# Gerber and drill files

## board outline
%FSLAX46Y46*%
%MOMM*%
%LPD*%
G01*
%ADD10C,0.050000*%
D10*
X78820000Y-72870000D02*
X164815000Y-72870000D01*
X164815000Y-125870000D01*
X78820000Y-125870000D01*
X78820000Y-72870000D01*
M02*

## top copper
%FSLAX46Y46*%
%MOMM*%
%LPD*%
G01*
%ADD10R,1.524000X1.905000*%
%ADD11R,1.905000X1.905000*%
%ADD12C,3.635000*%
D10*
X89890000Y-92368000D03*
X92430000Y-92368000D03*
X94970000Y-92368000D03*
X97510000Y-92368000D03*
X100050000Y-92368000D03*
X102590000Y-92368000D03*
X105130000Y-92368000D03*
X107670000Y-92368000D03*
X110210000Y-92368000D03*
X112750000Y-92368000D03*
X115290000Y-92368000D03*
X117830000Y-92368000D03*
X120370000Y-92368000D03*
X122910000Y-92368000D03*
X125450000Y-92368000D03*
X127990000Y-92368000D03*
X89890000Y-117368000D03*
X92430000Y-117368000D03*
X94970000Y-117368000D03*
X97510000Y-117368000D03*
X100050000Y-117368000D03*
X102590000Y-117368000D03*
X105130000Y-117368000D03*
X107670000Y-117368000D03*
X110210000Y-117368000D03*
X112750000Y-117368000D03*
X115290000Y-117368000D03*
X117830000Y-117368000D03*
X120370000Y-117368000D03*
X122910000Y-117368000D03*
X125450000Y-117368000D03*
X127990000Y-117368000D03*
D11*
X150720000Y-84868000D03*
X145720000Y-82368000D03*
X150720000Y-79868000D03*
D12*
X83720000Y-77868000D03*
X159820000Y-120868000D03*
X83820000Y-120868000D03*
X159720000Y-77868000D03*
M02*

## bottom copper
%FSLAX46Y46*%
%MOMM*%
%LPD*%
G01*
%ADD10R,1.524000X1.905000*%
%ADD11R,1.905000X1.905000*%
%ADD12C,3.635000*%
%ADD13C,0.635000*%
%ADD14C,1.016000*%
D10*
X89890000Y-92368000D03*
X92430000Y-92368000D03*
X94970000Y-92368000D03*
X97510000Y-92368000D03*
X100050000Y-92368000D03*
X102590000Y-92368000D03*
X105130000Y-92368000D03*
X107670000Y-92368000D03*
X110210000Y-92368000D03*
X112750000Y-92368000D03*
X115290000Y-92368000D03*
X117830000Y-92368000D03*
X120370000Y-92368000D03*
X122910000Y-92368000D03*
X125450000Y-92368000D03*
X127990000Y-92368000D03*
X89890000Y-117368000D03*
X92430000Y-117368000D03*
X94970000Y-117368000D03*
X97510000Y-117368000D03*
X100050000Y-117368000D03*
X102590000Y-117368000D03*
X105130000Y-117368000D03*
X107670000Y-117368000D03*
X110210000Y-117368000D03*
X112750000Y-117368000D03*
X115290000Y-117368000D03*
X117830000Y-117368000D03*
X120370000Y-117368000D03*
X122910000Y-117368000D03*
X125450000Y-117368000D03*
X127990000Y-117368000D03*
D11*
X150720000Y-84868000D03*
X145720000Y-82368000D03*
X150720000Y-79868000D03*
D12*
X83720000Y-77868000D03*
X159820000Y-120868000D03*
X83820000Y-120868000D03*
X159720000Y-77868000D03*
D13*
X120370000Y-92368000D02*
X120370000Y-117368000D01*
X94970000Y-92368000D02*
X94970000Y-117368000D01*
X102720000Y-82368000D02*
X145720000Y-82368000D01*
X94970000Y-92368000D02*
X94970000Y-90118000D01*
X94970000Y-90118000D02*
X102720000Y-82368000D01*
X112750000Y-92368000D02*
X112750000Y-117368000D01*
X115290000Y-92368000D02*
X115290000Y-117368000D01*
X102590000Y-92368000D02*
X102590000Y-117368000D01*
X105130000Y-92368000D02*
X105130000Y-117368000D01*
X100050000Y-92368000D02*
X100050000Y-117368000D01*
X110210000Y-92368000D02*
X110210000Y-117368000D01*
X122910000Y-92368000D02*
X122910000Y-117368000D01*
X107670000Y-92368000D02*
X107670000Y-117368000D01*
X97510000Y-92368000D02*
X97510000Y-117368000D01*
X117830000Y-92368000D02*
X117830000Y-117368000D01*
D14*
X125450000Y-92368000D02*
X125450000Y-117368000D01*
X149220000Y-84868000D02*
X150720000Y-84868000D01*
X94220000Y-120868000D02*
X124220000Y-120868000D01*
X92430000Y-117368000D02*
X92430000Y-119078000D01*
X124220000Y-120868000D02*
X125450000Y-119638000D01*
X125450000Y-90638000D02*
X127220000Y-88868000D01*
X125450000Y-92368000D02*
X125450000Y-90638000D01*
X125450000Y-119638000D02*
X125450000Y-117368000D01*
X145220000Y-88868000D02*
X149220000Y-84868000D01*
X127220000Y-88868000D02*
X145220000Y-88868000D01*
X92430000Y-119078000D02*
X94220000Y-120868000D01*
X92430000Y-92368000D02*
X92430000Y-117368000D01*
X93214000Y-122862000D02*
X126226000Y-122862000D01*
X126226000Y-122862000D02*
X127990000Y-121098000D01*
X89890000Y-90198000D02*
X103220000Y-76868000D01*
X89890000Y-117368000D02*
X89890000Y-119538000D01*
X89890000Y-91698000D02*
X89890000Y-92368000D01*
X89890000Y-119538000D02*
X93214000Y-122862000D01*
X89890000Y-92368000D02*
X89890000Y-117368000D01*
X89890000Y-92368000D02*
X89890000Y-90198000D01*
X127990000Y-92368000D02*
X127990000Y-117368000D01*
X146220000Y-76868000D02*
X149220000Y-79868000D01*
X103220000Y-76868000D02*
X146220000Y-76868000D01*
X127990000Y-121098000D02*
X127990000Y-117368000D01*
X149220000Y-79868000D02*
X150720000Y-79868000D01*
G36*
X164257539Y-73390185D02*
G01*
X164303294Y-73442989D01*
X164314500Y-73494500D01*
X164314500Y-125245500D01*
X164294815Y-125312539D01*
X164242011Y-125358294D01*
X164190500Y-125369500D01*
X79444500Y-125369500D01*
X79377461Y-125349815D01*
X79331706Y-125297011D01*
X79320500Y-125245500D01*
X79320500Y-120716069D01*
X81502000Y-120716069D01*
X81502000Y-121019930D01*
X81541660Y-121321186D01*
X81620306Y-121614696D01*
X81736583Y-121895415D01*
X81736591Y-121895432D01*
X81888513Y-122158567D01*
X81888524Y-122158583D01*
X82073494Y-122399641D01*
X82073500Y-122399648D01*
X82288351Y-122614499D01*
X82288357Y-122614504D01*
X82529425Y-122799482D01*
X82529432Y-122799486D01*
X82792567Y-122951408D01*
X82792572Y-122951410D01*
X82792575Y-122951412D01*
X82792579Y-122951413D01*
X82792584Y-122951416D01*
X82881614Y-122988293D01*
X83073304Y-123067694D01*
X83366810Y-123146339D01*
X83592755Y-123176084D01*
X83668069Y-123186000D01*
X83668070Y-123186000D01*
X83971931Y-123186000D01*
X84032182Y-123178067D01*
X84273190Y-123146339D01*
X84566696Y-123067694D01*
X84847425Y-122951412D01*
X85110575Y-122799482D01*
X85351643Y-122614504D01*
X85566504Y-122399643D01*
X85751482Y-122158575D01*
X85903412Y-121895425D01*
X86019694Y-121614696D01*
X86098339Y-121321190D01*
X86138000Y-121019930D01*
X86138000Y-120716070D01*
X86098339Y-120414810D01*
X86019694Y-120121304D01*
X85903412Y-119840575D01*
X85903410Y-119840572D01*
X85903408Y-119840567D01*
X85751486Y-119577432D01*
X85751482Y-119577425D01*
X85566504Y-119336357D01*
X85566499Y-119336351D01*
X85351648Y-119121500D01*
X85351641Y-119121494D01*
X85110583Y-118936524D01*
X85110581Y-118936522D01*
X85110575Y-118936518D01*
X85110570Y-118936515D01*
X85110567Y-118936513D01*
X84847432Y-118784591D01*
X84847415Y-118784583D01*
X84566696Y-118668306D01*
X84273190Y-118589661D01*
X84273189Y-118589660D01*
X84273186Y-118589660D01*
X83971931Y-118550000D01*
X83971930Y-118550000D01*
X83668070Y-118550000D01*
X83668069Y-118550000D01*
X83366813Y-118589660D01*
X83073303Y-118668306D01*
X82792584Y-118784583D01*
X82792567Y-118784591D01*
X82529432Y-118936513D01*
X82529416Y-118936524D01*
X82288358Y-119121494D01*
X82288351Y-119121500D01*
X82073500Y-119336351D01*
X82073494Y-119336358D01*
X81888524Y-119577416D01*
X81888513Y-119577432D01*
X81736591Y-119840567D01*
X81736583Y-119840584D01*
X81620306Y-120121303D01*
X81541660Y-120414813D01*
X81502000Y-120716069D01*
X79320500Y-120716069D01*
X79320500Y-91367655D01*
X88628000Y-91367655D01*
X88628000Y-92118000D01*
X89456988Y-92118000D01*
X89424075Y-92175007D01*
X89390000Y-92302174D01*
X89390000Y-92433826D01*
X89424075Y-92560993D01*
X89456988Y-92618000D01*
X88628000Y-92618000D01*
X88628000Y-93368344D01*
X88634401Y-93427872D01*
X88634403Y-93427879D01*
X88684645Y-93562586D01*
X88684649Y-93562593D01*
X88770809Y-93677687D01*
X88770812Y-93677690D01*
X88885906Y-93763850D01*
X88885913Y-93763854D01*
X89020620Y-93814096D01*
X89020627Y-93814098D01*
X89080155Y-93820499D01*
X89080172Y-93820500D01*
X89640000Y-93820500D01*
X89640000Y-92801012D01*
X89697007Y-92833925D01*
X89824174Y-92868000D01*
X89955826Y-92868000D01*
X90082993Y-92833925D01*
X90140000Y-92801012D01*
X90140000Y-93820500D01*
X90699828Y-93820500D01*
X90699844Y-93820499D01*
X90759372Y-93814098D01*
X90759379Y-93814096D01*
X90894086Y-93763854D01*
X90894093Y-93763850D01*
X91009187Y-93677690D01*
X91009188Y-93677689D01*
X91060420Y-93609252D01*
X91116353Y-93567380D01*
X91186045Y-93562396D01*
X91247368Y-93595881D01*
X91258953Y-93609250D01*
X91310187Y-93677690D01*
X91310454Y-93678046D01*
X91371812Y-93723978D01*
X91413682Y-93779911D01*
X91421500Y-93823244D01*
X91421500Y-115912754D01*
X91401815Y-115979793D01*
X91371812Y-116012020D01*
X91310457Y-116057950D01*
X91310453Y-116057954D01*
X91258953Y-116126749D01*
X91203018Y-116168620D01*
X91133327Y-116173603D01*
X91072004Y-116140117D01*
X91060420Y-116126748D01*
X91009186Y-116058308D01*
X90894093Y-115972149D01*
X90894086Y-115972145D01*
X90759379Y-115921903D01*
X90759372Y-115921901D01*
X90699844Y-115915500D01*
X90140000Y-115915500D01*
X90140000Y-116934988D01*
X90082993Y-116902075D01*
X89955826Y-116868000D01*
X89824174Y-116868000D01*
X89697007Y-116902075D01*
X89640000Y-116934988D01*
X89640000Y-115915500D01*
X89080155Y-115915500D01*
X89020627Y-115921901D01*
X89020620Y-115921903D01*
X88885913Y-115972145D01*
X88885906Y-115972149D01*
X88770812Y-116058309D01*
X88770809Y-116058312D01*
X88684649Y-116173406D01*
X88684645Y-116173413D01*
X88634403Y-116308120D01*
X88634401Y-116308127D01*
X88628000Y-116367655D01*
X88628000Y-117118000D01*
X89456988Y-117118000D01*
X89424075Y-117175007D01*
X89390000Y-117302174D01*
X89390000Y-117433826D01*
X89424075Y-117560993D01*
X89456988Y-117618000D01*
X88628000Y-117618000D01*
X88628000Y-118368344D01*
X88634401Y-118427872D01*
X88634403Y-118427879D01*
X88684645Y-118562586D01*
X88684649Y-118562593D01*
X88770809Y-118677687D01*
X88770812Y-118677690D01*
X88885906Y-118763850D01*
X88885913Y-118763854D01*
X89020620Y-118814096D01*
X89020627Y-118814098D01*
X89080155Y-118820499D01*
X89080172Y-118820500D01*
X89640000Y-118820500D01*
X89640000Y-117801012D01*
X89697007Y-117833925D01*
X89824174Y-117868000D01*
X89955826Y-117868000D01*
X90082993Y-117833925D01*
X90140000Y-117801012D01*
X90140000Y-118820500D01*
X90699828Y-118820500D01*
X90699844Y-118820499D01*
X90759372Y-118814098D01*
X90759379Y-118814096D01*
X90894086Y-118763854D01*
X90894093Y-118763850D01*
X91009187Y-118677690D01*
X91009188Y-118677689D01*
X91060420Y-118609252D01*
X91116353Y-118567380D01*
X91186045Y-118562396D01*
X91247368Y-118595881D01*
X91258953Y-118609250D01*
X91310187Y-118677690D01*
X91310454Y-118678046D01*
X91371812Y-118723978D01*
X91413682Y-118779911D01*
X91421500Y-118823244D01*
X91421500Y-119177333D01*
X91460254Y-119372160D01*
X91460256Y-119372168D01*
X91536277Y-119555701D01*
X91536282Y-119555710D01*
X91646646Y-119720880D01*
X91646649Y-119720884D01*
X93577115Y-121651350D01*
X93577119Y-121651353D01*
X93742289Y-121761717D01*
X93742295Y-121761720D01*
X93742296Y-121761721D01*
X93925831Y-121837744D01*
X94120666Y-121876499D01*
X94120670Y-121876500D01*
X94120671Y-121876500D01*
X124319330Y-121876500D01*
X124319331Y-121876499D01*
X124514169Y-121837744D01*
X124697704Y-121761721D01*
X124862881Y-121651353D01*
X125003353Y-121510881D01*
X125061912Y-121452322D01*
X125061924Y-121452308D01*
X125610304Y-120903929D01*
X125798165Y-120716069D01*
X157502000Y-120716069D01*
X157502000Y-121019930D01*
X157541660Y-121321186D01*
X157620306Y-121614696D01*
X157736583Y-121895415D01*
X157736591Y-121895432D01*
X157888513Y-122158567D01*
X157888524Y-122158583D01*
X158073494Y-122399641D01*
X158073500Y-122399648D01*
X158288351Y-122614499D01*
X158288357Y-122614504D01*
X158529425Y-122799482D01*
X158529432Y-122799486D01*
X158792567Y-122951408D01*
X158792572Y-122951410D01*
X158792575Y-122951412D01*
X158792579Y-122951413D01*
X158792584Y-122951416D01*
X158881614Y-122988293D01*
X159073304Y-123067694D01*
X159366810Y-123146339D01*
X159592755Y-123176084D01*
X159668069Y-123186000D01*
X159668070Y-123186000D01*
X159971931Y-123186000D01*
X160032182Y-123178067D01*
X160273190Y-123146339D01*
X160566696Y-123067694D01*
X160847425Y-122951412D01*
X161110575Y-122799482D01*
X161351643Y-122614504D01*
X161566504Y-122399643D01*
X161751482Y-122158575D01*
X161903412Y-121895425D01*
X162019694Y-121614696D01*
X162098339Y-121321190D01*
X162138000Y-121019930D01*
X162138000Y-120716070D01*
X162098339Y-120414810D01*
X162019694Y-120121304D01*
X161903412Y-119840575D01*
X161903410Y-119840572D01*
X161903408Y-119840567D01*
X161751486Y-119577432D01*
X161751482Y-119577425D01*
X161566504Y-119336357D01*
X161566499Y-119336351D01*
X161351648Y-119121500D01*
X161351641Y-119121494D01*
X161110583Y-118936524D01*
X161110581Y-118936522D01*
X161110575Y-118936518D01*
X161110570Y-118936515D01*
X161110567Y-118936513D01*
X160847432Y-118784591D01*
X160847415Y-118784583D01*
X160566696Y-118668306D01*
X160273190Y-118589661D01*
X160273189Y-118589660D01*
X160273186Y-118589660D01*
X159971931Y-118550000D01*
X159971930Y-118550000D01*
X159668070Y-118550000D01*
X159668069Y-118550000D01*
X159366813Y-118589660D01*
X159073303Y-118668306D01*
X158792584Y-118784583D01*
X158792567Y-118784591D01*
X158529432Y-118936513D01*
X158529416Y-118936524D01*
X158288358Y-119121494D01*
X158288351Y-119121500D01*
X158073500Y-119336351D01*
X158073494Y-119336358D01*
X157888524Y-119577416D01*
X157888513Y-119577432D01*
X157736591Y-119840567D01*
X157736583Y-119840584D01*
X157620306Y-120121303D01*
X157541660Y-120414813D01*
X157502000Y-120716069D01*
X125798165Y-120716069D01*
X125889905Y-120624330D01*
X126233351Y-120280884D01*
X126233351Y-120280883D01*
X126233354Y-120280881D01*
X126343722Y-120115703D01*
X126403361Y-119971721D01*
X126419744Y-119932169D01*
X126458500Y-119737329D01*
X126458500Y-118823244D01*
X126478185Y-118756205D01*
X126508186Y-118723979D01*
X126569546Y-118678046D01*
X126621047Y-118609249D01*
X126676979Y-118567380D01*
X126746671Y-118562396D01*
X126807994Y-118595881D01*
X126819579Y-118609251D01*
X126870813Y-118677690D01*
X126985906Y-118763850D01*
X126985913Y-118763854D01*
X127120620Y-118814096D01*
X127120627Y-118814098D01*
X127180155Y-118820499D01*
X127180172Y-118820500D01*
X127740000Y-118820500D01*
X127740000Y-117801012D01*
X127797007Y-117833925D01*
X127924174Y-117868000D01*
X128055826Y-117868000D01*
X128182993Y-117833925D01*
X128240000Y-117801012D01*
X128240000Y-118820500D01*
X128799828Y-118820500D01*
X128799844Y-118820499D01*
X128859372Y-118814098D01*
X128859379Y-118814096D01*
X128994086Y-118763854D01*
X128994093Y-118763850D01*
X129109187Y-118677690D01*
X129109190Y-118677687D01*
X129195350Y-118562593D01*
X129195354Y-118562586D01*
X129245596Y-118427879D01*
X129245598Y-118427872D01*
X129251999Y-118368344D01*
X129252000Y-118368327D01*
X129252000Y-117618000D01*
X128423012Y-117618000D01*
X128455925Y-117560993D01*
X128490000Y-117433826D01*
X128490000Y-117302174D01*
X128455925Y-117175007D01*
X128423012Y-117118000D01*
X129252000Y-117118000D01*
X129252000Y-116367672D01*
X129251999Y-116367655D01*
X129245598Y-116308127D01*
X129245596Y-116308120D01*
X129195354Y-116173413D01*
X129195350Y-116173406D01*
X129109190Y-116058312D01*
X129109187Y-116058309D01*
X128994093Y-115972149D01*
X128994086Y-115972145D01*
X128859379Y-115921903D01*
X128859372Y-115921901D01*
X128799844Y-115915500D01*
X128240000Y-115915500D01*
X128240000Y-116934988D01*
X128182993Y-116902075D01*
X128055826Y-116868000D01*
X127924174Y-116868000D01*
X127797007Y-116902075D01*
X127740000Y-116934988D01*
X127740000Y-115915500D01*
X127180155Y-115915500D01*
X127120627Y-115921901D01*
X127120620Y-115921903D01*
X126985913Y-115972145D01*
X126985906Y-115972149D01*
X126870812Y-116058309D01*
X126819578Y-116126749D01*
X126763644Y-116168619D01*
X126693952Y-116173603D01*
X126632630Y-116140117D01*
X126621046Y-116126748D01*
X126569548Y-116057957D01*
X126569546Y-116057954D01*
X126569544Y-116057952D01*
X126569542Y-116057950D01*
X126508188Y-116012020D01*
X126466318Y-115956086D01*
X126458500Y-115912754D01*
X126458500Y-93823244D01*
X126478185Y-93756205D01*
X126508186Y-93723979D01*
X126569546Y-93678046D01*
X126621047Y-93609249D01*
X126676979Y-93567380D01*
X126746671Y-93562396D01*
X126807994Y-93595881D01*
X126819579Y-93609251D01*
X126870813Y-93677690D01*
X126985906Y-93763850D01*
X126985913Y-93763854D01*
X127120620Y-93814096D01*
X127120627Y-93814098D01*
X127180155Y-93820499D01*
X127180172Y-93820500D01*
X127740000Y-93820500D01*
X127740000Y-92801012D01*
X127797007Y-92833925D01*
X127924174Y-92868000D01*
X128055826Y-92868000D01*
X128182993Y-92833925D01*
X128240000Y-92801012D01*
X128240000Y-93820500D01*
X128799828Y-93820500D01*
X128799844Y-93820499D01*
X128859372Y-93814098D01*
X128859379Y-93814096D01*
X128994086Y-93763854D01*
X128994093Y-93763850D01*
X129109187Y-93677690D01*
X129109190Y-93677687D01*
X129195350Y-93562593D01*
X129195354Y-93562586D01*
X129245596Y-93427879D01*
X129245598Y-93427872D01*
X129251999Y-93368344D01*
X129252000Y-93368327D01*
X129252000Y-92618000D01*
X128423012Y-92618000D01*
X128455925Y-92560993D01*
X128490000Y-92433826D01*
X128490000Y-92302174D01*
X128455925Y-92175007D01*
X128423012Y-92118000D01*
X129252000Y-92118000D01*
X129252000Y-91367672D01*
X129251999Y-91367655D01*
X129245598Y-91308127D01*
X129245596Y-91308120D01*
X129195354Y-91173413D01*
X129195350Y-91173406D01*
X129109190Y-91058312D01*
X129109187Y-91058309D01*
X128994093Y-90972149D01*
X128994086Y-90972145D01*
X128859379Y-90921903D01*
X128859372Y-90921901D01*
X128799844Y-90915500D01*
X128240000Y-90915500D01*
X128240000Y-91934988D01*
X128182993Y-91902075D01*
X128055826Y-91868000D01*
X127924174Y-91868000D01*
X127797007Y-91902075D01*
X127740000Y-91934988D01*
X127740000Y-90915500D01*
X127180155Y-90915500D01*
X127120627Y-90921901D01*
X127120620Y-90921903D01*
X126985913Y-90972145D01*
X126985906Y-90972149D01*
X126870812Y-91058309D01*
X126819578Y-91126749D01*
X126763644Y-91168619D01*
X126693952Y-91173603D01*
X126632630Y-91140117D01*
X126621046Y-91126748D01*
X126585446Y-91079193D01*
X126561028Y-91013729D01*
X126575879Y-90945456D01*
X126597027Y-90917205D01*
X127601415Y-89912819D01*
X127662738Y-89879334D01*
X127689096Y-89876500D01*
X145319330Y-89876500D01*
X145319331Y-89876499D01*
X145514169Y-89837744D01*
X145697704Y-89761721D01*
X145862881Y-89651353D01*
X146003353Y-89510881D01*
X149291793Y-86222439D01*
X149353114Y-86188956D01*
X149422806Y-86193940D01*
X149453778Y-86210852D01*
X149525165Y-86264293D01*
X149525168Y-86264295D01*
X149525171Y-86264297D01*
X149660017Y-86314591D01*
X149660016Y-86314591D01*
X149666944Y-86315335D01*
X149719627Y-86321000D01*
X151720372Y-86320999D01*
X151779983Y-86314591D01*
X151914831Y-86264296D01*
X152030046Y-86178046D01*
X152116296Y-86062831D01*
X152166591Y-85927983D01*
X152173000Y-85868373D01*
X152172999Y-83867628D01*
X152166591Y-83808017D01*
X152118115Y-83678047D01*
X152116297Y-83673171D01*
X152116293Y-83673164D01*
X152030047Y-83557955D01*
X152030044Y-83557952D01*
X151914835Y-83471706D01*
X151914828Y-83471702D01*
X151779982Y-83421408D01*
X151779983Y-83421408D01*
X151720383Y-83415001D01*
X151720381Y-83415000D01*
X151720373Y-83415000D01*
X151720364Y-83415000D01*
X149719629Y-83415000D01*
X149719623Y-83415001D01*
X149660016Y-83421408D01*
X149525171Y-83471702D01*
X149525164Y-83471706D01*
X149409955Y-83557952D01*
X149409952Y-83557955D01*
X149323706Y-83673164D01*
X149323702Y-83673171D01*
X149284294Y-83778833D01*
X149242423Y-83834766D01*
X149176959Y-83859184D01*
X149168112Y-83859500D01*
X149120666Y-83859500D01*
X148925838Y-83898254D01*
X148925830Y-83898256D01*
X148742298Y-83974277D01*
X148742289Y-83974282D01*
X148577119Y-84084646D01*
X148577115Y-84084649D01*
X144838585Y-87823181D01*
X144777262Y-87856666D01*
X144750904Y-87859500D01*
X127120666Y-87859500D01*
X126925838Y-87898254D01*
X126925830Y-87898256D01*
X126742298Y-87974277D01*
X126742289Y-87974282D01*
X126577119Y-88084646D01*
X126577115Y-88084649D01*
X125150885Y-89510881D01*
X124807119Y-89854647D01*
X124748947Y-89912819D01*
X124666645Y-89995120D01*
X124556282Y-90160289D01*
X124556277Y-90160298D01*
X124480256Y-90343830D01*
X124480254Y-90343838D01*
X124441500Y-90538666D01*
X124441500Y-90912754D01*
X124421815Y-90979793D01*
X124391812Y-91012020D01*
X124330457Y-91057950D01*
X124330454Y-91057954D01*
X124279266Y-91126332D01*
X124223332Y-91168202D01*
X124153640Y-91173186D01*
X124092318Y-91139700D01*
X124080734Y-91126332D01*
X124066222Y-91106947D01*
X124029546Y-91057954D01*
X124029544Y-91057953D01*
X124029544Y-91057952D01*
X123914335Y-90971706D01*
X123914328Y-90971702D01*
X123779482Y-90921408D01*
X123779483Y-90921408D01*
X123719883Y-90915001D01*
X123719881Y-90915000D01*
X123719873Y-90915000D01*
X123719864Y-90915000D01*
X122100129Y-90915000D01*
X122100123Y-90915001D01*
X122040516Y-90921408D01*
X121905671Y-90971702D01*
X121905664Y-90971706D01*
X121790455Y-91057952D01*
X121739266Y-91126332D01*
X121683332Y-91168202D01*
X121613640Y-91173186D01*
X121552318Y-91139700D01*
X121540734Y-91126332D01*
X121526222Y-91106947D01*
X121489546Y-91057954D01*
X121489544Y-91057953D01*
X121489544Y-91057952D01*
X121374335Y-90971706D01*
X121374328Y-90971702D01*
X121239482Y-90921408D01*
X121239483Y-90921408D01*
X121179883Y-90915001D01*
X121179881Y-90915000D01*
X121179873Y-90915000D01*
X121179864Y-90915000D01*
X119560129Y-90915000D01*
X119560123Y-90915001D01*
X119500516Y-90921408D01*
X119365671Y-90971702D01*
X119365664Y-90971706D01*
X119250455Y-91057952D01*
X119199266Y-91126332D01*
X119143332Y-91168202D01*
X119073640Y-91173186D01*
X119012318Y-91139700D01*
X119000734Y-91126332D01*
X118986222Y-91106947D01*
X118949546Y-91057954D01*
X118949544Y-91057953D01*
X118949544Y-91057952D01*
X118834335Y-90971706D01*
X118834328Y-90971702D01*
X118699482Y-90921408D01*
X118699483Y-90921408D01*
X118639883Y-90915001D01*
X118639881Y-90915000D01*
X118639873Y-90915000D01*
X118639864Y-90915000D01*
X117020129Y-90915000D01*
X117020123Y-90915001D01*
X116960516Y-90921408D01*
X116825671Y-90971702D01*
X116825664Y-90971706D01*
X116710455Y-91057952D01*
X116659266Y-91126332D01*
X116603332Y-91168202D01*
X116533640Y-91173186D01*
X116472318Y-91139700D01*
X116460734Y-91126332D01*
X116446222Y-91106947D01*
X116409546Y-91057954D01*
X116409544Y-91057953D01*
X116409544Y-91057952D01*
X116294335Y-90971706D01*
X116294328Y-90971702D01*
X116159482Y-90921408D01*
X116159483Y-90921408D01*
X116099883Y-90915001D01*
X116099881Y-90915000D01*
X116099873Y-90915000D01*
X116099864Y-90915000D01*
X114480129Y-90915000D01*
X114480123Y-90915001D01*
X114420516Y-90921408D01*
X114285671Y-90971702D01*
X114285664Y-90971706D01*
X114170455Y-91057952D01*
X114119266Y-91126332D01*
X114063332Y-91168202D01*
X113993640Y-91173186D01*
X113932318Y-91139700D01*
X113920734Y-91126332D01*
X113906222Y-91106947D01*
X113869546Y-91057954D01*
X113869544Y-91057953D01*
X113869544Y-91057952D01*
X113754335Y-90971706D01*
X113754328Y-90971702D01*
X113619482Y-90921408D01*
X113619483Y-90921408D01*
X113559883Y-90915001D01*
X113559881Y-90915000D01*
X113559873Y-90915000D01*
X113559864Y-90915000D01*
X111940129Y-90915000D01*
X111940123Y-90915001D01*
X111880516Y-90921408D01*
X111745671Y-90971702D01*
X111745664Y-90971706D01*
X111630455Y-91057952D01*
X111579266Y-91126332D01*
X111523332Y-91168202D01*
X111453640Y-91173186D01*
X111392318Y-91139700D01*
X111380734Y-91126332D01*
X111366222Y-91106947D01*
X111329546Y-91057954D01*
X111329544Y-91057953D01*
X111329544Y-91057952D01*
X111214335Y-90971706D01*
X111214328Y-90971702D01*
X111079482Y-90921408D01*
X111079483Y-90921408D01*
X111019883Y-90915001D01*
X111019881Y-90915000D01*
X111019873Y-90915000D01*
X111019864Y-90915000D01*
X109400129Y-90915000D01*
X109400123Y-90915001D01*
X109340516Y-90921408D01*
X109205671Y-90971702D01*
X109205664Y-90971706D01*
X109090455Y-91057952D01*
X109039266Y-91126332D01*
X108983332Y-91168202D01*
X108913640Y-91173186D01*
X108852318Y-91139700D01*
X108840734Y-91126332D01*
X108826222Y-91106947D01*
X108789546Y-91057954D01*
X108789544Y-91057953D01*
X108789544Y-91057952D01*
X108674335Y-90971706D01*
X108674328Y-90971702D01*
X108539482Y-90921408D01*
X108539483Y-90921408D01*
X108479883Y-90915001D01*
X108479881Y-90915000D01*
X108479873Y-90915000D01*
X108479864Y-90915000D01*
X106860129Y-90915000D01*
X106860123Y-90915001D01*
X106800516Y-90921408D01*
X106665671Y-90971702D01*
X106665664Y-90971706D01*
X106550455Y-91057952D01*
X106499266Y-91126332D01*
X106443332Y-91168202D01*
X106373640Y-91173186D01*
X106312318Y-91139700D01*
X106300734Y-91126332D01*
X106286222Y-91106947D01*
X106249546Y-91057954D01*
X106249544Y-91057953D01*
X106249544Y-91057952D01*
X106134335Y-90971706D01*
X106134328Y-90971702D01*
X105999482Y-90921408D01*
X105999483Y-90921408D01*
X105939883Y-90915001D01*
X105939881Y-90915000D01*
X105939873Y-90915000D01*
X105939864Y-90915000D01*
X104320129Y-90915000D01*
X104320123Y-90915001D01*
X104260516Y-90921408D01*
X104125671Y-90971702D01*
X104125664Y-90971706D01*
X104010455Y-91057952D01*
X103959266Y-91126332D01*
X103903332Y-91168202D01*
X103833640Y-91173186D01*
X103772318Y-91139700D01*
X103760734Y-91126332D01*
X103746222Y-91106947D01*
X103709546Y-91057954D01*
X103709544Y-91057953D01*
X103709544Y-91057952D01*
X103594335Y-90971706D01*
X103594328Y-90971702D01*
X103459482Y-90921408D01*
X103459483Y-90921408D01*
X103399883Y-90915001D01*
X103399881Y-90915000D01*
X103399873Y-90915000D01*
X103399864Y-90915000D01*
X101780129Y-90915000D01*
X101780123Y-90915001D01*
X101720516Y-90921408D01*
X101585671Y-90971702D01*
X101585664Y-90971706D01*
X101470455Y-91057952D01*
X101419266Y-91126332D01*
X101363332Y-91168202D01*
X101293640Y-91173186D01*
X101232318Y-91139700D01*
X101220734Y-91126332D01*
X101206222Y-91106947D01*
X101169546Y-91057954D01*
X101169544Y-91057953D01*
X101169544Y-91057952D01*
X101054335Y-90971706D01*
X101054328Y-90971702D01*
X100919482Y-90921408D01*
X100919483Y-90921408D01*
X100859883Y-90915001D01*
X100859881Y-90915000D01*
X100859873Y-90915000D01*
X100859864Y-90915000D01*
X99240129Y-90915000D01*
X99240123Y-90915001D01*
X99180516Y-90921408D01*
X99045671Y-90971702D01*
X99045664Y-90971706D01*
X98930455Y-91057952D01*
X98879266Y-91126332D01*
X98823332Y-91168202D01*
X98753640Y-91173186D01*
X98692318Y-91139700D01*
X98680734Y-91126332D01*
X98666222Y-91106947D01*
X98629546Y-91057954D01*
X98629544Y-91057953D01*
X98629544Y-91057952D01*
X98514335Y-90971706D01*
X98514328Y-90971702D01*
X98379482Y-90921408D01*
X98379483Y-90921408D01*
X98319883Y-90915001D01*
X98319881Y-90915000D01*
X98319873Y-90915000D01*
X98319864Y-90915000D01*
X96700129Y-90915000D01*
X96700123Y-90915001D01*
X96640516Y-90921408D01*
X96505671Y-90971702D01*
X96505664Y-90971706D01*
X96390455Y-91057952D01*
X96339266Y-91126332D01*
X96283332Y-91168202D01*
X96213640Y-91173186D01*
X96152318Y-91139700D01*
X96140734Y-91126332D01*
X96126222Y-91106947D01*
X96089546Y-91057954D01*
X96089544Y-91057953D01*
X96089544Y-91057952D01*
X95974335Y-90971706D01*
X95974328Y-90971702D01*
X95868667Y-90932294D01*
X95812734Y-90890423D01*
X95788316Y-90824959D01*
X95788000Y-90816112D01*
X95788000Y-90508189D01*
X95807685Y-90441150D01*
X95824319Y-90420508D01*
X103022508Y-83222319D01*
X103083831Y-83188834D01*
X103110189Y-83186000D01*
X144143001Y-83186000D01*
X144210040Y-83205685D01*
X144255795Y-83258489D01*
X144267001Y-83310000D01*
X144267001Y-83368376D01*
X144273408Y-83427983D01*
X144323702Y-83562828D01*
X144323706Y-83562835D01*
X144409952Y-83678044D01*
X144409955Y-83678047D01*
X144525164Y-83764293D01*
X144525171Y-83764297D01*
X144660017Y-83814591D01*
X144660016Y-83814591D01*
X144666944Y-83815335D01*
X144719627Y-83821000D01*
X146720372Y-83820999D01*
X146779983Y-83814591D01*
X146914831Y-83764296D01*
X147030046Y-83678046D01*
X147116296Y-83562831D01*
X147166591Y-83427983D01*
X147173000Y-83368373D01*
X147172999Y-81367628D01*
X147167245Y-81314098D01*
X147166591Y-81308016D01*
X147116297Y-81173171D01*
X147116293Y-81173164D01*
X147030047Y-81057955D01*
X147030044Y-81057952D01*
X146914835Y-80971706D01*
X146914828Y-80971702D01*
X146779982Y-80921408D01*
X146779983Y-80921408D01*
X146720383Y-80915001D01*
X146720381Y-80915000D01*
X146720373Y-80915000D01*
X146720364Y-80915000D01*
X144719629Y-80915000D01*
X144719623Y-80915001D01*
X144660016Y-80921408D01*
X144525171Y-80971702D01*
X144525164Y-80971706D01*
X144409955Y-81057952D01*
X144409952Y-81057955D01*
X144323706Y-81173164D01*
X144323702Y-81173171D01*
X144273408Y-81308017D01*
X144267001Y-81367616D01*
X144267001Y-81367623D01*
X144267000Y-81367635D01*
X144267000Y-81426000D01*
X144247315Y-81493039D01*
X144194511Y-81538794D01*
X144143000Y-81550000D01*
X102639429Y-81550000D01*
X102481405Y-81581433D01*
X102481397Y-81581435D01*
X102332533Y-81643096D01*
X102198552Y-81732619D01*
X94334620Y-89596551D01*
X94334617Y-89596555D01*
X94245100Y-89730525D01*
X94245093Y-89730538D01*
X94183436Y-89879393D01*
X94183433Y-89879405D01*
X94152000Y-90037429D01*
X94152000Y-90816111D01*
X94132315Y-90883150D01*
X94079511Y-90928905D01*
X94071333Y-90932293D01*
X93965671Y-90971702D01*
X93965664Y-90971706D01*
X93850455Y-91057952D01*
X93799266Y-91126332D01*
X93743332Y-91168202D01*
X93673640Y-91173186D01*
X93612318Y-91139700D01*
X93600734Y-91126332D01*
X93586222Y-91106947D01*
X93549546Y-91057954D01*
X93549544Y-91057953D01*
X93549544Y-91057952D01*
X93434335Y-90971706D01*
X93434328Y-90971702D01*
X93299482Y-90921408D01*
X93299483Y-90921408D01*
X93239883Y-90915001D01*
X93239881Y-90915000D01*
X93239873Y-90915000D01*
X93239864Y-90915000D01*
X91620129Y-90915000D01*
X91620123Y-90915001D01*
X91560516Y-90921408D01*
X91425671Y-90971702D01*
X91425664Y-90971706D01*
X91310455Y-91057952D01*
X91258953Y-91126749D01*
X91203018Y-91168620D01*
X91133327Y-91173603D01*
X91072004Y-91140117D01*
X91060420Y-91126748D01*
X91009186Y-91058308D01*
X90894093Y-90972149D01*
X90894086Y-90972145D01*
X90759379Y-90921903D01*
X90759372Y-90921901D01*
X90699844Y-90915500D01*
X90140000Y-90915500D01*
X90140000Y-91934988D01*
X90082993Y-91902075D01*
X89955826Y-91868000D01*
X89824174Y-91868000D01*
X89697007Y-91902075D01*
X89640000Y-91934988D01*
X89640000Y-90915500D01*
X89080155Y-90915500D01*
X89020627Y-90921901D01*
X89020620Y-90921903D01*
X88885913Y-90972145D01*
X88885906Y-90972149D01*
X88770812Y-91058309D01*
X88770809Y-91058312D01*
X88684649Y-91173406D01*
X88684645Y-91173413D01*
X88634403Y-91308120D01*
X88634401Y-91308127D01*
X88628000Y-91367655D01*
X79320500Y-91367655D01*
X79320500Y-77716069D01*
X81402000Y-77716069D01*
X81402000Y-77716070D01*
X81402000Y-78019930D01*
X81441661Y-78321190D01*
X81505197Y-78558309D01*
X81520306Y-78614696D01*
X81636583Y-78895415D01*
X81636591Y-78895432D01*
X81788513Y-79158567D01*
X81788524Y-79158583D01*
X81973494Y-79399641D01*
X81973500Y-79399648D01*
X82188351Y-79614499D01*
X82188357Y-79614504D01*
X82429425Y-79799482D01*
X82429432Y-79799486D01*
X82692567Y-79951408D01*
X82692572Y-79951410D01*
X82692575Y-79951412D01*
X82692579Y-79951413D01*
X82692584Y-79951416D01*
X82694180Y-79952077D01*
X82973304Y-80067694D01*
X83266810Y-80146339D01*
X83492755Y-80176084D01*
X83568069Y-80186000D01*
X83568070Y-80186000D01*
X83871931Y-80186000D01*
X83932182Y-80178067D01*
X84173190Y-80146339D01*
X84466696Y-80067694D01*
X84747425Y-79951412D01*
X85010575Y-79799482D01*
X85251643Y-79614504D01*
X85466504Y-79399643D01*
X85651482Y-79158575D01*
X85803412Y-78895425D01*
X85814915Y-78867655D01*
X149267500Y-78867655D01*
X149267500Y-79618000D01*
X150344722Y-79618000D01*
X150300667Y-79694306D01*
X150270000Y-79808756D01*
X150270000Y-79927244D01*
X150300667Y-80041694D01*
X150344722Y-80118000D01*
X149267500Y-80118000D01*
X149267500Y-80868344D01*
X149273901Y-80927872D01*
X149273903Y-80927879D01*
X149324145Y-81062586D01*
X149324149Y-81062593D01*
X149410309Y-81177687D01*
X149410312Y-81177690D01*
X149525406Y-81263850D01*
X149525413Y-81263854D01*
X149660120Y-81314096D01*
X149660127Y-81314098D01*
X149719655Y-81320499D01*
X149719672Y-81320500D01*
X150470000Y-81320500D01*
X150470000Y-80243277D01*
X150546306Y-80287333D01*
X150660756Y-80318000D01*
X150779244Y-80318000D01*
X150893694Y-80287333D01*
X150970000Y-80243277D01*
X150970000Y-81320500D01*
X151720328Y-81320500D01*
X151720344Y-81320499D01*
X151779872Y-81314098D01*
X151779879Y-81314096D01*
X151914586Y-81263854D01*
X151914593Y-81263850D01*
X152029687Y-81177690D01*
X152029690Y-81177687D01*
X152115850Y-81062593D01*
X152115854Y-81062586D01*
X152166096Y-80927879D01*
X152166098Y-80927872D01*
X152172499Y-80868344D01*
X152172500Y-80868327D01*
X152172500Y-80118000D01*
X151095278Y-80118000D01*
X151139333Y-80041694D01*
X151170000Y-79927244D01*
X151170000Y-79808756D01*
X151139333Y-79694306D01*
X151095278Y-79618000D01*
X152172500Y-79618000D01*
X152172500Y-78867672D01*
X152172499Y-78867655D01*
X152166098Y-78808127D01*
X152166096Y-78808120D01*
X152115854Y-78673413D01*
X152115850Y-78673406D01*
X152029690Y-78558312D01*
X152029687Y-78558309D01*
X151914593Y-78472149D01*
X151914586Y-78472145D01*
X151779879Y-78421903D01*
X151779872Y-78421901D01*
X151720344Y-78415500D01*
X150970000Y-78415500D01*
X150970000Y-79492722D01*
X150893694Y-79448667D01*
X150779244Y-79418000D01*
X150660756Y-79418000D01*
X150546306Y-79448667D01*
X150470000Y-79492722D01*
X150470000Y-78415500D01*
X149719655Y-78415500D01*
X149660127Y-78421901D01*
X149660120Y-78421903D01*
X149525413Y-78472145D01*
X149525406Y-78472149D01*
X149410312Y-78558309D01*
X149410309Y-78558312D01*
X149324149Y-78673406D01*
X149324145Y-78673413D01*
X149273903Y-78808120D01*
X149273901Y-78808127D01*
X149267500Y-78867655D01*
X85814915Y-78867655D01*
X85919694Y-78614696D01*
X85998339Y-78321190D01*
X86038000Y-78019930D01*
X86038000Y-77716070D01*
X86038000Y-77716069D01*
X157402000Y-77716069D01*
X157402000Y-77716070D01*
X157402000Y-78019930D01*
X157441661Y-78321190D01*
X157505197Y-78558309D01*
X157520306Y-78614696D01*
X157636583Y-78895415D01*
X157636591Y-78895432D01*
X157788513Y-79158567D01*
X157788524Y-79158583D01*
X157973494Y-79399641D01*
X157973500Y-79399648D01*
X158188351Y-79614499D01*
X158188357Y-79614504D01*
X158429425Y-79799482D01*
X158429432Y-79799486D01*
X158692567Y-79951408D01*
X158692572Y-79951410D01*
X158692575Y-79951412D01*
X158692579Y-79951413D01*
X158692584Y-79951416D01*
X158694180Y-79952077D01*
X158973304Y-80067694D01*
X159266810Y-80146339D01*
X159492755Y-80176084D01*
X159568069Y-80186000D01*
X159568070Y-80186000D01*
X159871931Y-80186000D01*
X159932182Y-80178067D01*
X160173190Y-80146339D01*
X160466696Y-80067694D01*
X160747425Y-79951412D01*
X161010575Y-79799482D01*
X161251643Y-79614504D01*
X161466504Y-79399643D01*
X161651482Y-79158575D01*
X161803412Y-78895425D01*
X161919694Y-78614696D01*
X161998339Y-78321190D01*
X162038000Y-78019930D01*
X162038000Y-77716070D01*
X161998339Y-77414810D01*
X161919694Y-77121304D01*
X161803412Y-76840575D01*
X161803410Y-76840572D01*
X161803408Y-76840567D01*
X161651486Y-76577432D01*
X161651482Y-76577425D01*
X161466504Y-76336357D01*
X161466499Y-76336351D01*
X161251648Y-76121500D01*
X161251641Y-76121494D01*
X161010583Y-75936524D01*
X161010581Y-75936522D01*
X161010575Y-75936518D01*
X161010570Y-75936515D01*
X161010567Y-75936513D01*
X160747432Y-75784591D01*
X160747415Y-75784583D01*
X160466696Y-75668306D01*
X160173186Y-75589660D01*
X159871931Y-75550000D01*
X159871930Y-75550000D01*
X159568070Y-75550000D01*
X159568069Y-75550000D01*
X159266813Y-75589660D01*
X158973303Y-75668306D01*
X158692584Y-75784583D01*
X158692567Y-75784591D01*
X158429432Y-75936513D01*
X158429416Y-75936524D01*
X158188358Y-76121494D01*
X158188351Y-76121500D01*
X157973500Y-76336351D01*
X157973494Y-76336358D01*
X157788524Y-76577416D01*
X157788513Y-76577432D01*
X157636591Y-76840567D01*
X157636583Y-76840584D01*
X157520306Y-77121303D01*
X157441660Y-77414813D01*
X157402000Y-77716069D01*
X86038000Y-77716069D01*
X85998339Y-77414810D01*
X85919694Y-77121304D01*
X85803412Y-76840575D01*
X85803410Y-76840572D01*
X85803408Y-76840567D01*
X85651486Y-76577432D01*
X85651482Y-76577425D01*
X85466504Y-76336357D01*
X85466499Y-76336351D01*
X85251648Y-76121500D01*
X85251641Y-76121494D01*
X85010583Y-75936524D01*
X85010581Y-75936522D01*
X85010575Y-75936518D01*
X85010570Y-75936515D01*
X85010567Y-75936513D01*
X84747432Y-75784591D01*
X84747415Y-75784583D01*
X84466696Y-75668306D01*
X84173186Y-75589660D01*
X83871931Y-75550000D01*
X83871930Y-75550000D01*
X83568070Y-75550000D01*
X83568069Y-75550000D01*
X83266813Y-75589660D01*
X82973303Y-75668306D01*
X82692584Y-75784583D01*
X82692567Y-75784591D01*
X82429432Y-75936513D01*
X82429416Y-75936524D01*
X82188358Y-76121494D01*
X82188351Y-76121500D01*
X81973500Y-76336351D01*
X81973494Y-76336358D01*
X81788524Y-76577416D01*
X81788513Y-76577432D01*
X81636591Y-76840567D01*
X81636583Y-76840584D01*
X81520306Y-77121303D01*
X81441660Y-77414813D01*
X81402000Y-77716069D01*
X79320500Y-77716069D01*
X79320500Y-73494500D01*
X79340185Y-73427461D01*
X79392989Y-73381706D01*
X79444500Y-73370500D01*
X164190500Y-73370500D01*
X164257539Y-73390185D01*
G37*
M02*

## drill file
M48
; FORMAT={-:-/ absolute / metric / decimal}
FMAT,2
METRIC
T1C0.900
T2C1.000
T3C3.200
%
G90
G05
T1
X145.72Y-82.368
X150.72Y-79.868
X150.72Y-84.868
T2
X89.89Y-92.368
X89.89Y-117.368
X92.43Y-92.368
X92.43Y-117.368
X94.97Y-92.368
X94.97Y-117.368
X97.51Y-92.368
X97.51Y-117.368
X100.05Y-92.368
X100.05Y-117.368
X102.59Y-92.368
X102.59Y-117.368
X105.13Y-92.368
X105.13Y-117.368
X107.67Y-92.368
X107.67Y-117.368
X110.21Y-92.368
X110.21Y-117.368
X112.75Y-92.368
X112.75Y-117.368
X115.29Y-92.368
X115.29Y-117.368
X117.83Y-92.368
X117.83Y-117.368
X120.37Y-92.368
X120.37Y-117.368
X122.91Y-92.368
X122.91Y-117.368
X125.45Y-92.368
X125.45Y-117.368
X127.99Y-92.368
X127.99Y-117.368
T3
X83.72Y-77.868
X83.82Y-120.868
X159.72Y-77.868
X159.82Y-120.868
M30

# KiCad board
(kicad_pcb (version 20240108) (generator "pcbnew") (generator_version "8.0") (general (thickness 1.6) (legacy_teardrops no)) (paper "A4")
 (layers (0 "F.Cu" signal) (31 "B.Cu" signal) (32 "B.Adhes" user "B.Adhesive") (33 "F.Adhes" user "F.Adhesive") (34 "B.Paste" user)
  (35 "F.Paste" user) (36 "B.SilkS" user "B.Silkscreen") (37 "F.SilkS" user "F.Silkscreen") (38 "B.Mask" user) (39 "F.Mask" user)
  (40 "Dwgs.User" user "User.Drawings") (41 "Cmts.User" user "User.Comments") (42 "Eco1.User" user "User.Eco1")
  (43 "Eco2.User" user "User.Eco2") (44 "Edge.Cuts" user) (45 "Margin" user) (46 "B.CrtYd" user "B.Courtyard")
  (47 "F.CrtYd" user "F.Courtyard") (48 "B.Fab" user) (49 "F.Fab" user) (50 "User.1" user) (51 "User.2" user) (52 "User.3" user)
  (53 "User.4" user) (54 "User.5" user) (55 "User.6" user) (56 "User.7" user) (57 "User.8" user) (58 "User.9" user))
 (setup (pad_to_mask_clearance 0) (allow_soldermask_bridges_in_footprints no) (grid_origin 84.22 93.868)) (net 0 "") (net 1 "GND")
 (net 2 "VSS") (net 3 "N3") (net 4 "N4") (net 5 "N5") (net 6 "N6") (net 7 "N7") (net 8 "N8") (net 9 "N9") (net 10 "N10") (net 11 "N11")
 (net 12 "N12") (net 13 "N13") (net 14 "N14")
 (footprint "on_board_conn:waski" (layer "F.Cu") (at 89.89 92.368 90)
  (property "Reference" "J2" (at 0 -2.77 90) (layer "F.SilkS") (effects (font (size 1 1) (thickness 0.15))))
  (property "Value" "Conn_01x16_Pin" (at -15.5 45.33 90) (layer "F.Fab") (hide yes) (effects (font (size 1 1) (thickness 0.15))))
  (pad "1" thru_hole rect (at 0 0 90) (size 1.905 1.524) (drill 1) (layers "*.Cu" "*.Mask") (remove_unused_layers no) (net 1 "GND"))
  (pad "2" thru_hole rect (at 0 2.54 90) (size 1.905 1.524) (drill 1) (layers "*.Cu" "*.Mask") (remove_unused_layers no) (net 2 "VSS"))
  (pad "3" thru_hole rect (at 0 5.08 90) (size 1.905 1.524) (drill 1) (layers "*.Cu" "*.Mask") (remove_unused_layers no) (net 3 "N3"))
  (pad "4" thru_hole rect (at 0 7.62 90) (size 1.905 1.524) (drill 1) (layers "*.Cu" "*.Mask") (remove_unused_layers no) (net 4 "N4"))
  (pad "5" thru_hole rect (at 0 10.16 90) (size 1.905 1.524) (drill 1) (layers "*.Cu" "*.Mask") (remove_unused_layers no) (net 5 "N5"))
  (pad "6" thru_hole rect (at 0 12.7 90) (size 1.905 1.524) (drill 1) (layers "*.Cu" "*.Mask") (remove_unused_layers no) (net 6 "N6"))
  (pad "7" thru_hole rect (at 0 15.24 90) (size 1.905 1.524) (drill 1) (layers "*.Cu" "*.Mask") (remove_unused_layers no) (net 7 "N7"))
  (pad "8" thru_hole rect (at 0 17.78 90) (size 1.905 1.524) (drill 1) (layers "*.Cu" "*.Mask") (remove_unused_layers no) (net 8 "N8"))
  (pad "9" thru_hole rect (at 0 20.32 90) (size 1.905 1.524) (drill 1) (layers "*.Cu" "*.Mask") (remove_unused_layers no) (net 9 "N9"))
  (pad "10" thru_hole rect (at 0 22.86 90) (size 1.905 1.524) (drill 1) (layers "*.Cu" "*.Mask") (remove_unused_layers no) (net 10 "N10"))
  (pad "11" thru_hole rect (at 0 25.4 90) (size 1.905 1.524) (drill 1) (layers "*.Cu" "*.Mask") (remove_unused_layers no) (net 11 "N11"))
  (pad "12" thru_hole rect (at 0 27.94 90) (size 1.905 1.524) (drill 1) (layers "*.Cu" "*.Mask") (remove_unused_layers no) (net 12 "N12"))
  (pad "13" thru_hole rect (at 0 30.48 90) (size 1.905 1.524) (drill 1) (layers "*.Cu" "*.Mask") (remove_unused_layers no) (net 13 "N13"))
  (pad "14" thru_hole rect (at 0 33.02 90) (size 1.905 1.524) (drill 1) (layers "*.Cu" "*.Mask") (remove_unused_layers no) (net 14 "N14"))
  (pad "15" thru_hole rect (at 0 35.56 90) (size 1.905 1.524) (drill 1) (layers "*.Cu" "*.Mask") (remove_unused_layers no) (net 2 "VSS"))
  (pad "16" thru_hole rect (at 0 38.1 90) (size 1.905 1.524) (drill 1) (layers "*.Cu" "*.Mask") (remove_unused_layers no) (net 1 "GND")))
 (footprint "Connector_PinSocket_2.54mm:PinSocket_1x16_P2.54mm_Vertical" (layer "F.Cu") (at 89.89 117.368 90)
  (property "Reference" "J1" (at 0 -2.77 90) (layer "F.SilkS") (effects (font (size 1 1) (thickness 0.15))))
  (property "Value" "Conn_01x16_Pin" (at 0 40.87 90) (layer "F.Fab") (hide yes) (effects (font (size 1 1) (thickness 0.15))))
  (pad "1" thru_hole rect (at 0 0 90) (size 1.905 1.524) (drill 1) (layers "*.Cu" "*.Mask") (remove_unused_layers no) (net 1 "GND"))
  (pad "2" thru_hole rect (at 0 2.54 90) (size 1.905 1.524) (drill 1) (layers "*.Cu" "*.Mask") (remove_unused_layers no) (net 2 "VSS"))
  (pad "3" thru_hole rect (at 0 5.08 90) (size 1.905 1.524) (drill 1) (layers "*.Cu" "*.Mask") (remove_unused_layers no) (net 3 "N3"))
  (pad "4" thru_hole rect (at 0 7.62 90) (size 1.905 1.524) (drill 1) (layers "*.Cu" "*.Mask") (remove_unused_layers no) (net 4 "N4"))
  (pad "5" thru_hole rect (at 0 10.16 90) (size 1.905 1.524) (drill 1) (layers "*.Cu" "*.Mask") (remove_unused_layers no) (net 5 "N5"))
  (pad "6" thru_hole rect (at 0 12.7 90) (size 1.905 1.524) (drill 1) (layers "*.Cu" "*.Mask") (remove_unused_layers no) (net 6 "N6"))
  (pad "7" thru_hole rect (at 0 15.24 90) (size 1.905 1.524) (drill 1) (layers "*.Cu" "*.Mask") (remove_unused_layers no) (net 7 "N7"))
  (pad "8" thru_hole rect (at 0 17.78 90) (size 1.905 1.524) (drill 1) (layers "*.Cu" "*.Mask") (remove_unused_layers no) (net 8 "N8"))
  (pad "9" thru_hole rect (at 0 20.32 90) (size 1.905 1.524) (drill 1) (layers "*.Cu" "*.Mask") (remove_unused_layers no) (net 9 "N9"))
  (pad "10" thru_hole rect (at 0 22.86 90) (size 1.905 1.524) (drill 1) (layers "*.Cu" "*.Mask") (remove_unused_layers no) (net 10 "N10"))
  (pad "11" thru_hole rect (at 0 25.4 90) (size 1.905 1.524) (drill 1) (layers "*.Cu" "*.Mask") (remove_unused_layers no) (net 11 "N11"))
  (pad "12" thru_hole rect (at 0 27.94 90) (size 1.905 1.524) (drill 1) (layers "*.Cu" "*.Mask") (remove_unused_layers no) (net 12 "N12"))
  (pad "13" thru_hole rect (at 0 30.48 90) (size 1.905 1.524) (drill 1) (layers "*.Cu" "*.Mask") (remove_unused_layers no) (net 13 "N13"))
  (pad "14" thru_hole rect (at 0 33.02 90) (size 1.905 1.524) (drill 1) (layers "*.Cu" "*.Mask") (remove_unused_layers no) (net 14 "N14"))
  (pad "15" thru_hole rect (at 0 35.56 90) (size 1.905 1.524) (drill 1) (layers "*.Cu" "*.Mask") (remove_unused_layers no) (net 2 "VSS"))
  (pad "16" thru_hole rect (at 0 38.1 90) (size 1.905 1.524) (drill 1) (layers "*.Cu" "*.Mask") (remove_unused_layers no) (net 1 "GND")))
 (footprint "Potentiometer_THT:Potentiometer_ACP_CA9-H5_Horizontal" (layer "F.Cu") (at 150.72 84.868 180)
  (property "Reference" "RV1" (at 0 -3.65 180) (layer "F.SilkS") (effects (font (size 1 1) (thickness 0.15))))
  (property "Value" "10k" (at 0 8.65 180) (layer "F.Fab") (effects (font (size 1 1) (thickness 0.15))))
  (pad "1" thru_hole rect (at 0 0 180) (size 1.905 1.905) (drill 0.9) (layers "*.Cu" "*.Mask") (remove_unused_layers no) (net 2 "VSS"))
  (pad "2" thru_hole rect (at 5 2.5 180) (size 1.905 1.905) (drill 0.9) (layers "*.Cu" "*.Mask") (remove_unused_layers no) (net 3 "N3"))
  (pad "3" thru_hole rect (at 0 5 180) (size 1.905 1.905) (drill 0.9) (layers "*.Cu" "*.Mask") (remove_unused_layers no) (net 1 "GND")))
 (gr_rect (start 78.82 72.87) (end 164.815 125.87) (stroke (width 0.05) (type default)) (fill none) (layer "Edge.Cuts"))
 (via (at 83.72 77.868) (size 3.635) (drill 3.2) (layers "F.Cu" "B.Cu") (free yes) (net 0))
 (via (at 159.82 120.868) (size 3.635) (drill 3.2) (layers "F.Cu" "B.Cu") (free yes) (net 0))
 (via (at 83.82 120.868) (size 3.635) (drill 3.2) (layers "F.Cu" "B.Cu") (free yes) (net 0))
 (via (at 159.72 77.868) (size 3.635) (drill 3.2) (layers "F.Cu" "B.Cu") (free yes) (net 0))
 (segment (start 120.37 92.368) (end 120.37 117.368) (width 0.635) (layer "B.Cu") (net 13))
 (segment (start 94.97 92.368) (end 94.97 117.368) (width 0.635) (layer "B.Cu") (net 3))
 (segment (start 102.72 82.368) (end 145.72 82.368) (width 0.635) (layer "B.Cu") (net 3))
 (segment (start 94.97 92.368) (end 94.97 90.118) (width 0.635) (layer "B.Cu") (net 3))
 (segment (start 94.97 90.118) (end 102.72 82.368) (width 0.635) (layer "B.Cu") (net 3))
 (segment (start 112.75 92.368) (end 112.75 117.368) (width 0.635) (layer "B.Cu") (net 10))
 (segment (start 115.29 92.368) (end 115.29 117.368) (width 0.635) (layer "B.Cu") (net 11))
 (segment (start 102.59 92.368) (end 102.59 117.368) (width 0.635) (layer "B.Cu") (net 6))
 (segment (start 105.13 92.368) (end 105.13 117.368) (width 0.635) (layer "B.Cu") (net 7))
 (segment (start 100.05 92.368) (end 100.05 117.368) (width 0.635) (layer "B.Cu") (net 5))
 (segment (start 110.21 92.368) (end 110.21 117.368) (width 0.635) (layer "B.Cu") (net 9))
 (segment (start 122.91 92.368) (end 122.91 117.368) (width 0.635) (layer "B.Cu") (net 14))
 (segment (start 107.67 92.368) (end 107.67 117.368) (width 0.635) (layer "B.Cu") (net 8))
 (segment (start 97.51 92.368) (end 97.51 117.368) (width 0.635) (layer "B.Cu") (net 4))
 (segment (start 117.83 92.368) (end 117.83 117.368) (width 0.635) (layer "B.Cu") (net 12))
 (segment (start 125.45 92.368) (end 125.45 117.368) (width 1.016) (layer "B.Cu") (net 2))
 (segment (start 149.22 84.868) (end 150.72 84.868) (width 1.016) (layer "B.Cu") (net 2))
 (segment (start 94.22 120.868) (end 124.22 120.868) (width 1.016) (layer "B.Cu") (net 2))
 (segment (start 92.43 117.368) (end 92.43 119.078) (width 1.016) (layer "B.Cu") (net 2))
 (segment (start 124.22 120.868) (end 125.45 119.638) (width 1.016) (layer "B.Cu") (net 2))
 (segment (start 125.45 90.638) (end 127.22 88.868) (width 1.016) (layer "B.Cu") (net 2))
 (segment (start 125.45 92.368) (end 125.45 90.638) (width 1.016) (layer "B.Cu") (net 2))
 (segment (start 125.45 119.638) (end 125.45 117.368) (width 1.016) (layer "B.Cu") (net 2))
 (segment (start 145.22 88.868) (end 149.22 84.868) (width 1.016) (layer "B.Cu") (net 2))
 (segment (start 127.22 88.868) (end 145.22 88.868) (width 1.016) (layer "B.Cu") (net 2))
 (segment (start 92.43 119.078) (end 94.22 120.868) (width 1.016) (layer "B.Cu") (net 2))
 (segment (start 92.43 92.368) (end 92.43 117.368) (width 1.016) (layer "B.Cu") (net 2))
 (segment (start 93.214 122.862) (end 126.226 122.862) (width 1.016) (layer "B.Cu") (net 1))
 (segment (start 126.226 122.862) (end 127.99 121.098) (width 1.016) (layer "B.Cu") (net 1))
 (segment (start 89.89 90.198) (end 103.22 76.868) (width 1.016) (layer "B.Cu") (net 1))
 (segment (start 89.89 117.368) (end 89.89 119.538) (width 1.016) (layer "B.Cu") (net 1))
 (segment (start 89.89 91.698) (end 89.89 92.368) (width 1.016) (layer "B.Cu") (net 1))
 (segment (start 89.89 119.538) (end 93.214 122.862) (width 1.016) (layer "B.Cu") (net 1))
 (segment (start 89.89 92.368) (end 89.89 117.368) (width 1.016) (layer "B.Cu") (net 1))
 (segment (start 89.89 92.368) (end 89.89 90.198) (width 1.016) (layer "B.Cu") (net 1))
 (segment (start 127.99 92.368) (end 127.99 117.368) (width 1.016) (layer "B.Cu") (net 1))
 (segment (start 146.22 76.868) (end 149.22 79.868) (width 1.016) (layer "B.Cu") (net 1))
 (segment (start 103.22 76.868) (end 146.22 76.868) (width 1.016) (layer "B.Cu") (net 1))
 (segment (start 127.99 121.098) (end 127.99 117.368) (width 1.016) (layer "B.Cu") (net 1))
 (segment (start 149.22 79.868) (end 150.72 79.868) (width 1.016) (layer "B.Cu") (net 1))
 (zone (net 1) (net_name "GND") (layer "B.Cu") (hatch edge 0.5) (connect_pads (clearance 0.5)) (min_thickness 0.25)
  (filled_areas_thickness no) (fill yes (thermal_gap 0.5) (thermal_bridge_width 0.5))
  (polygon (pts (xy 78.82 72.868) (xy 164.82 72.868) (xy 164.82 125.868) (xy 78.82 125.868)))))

